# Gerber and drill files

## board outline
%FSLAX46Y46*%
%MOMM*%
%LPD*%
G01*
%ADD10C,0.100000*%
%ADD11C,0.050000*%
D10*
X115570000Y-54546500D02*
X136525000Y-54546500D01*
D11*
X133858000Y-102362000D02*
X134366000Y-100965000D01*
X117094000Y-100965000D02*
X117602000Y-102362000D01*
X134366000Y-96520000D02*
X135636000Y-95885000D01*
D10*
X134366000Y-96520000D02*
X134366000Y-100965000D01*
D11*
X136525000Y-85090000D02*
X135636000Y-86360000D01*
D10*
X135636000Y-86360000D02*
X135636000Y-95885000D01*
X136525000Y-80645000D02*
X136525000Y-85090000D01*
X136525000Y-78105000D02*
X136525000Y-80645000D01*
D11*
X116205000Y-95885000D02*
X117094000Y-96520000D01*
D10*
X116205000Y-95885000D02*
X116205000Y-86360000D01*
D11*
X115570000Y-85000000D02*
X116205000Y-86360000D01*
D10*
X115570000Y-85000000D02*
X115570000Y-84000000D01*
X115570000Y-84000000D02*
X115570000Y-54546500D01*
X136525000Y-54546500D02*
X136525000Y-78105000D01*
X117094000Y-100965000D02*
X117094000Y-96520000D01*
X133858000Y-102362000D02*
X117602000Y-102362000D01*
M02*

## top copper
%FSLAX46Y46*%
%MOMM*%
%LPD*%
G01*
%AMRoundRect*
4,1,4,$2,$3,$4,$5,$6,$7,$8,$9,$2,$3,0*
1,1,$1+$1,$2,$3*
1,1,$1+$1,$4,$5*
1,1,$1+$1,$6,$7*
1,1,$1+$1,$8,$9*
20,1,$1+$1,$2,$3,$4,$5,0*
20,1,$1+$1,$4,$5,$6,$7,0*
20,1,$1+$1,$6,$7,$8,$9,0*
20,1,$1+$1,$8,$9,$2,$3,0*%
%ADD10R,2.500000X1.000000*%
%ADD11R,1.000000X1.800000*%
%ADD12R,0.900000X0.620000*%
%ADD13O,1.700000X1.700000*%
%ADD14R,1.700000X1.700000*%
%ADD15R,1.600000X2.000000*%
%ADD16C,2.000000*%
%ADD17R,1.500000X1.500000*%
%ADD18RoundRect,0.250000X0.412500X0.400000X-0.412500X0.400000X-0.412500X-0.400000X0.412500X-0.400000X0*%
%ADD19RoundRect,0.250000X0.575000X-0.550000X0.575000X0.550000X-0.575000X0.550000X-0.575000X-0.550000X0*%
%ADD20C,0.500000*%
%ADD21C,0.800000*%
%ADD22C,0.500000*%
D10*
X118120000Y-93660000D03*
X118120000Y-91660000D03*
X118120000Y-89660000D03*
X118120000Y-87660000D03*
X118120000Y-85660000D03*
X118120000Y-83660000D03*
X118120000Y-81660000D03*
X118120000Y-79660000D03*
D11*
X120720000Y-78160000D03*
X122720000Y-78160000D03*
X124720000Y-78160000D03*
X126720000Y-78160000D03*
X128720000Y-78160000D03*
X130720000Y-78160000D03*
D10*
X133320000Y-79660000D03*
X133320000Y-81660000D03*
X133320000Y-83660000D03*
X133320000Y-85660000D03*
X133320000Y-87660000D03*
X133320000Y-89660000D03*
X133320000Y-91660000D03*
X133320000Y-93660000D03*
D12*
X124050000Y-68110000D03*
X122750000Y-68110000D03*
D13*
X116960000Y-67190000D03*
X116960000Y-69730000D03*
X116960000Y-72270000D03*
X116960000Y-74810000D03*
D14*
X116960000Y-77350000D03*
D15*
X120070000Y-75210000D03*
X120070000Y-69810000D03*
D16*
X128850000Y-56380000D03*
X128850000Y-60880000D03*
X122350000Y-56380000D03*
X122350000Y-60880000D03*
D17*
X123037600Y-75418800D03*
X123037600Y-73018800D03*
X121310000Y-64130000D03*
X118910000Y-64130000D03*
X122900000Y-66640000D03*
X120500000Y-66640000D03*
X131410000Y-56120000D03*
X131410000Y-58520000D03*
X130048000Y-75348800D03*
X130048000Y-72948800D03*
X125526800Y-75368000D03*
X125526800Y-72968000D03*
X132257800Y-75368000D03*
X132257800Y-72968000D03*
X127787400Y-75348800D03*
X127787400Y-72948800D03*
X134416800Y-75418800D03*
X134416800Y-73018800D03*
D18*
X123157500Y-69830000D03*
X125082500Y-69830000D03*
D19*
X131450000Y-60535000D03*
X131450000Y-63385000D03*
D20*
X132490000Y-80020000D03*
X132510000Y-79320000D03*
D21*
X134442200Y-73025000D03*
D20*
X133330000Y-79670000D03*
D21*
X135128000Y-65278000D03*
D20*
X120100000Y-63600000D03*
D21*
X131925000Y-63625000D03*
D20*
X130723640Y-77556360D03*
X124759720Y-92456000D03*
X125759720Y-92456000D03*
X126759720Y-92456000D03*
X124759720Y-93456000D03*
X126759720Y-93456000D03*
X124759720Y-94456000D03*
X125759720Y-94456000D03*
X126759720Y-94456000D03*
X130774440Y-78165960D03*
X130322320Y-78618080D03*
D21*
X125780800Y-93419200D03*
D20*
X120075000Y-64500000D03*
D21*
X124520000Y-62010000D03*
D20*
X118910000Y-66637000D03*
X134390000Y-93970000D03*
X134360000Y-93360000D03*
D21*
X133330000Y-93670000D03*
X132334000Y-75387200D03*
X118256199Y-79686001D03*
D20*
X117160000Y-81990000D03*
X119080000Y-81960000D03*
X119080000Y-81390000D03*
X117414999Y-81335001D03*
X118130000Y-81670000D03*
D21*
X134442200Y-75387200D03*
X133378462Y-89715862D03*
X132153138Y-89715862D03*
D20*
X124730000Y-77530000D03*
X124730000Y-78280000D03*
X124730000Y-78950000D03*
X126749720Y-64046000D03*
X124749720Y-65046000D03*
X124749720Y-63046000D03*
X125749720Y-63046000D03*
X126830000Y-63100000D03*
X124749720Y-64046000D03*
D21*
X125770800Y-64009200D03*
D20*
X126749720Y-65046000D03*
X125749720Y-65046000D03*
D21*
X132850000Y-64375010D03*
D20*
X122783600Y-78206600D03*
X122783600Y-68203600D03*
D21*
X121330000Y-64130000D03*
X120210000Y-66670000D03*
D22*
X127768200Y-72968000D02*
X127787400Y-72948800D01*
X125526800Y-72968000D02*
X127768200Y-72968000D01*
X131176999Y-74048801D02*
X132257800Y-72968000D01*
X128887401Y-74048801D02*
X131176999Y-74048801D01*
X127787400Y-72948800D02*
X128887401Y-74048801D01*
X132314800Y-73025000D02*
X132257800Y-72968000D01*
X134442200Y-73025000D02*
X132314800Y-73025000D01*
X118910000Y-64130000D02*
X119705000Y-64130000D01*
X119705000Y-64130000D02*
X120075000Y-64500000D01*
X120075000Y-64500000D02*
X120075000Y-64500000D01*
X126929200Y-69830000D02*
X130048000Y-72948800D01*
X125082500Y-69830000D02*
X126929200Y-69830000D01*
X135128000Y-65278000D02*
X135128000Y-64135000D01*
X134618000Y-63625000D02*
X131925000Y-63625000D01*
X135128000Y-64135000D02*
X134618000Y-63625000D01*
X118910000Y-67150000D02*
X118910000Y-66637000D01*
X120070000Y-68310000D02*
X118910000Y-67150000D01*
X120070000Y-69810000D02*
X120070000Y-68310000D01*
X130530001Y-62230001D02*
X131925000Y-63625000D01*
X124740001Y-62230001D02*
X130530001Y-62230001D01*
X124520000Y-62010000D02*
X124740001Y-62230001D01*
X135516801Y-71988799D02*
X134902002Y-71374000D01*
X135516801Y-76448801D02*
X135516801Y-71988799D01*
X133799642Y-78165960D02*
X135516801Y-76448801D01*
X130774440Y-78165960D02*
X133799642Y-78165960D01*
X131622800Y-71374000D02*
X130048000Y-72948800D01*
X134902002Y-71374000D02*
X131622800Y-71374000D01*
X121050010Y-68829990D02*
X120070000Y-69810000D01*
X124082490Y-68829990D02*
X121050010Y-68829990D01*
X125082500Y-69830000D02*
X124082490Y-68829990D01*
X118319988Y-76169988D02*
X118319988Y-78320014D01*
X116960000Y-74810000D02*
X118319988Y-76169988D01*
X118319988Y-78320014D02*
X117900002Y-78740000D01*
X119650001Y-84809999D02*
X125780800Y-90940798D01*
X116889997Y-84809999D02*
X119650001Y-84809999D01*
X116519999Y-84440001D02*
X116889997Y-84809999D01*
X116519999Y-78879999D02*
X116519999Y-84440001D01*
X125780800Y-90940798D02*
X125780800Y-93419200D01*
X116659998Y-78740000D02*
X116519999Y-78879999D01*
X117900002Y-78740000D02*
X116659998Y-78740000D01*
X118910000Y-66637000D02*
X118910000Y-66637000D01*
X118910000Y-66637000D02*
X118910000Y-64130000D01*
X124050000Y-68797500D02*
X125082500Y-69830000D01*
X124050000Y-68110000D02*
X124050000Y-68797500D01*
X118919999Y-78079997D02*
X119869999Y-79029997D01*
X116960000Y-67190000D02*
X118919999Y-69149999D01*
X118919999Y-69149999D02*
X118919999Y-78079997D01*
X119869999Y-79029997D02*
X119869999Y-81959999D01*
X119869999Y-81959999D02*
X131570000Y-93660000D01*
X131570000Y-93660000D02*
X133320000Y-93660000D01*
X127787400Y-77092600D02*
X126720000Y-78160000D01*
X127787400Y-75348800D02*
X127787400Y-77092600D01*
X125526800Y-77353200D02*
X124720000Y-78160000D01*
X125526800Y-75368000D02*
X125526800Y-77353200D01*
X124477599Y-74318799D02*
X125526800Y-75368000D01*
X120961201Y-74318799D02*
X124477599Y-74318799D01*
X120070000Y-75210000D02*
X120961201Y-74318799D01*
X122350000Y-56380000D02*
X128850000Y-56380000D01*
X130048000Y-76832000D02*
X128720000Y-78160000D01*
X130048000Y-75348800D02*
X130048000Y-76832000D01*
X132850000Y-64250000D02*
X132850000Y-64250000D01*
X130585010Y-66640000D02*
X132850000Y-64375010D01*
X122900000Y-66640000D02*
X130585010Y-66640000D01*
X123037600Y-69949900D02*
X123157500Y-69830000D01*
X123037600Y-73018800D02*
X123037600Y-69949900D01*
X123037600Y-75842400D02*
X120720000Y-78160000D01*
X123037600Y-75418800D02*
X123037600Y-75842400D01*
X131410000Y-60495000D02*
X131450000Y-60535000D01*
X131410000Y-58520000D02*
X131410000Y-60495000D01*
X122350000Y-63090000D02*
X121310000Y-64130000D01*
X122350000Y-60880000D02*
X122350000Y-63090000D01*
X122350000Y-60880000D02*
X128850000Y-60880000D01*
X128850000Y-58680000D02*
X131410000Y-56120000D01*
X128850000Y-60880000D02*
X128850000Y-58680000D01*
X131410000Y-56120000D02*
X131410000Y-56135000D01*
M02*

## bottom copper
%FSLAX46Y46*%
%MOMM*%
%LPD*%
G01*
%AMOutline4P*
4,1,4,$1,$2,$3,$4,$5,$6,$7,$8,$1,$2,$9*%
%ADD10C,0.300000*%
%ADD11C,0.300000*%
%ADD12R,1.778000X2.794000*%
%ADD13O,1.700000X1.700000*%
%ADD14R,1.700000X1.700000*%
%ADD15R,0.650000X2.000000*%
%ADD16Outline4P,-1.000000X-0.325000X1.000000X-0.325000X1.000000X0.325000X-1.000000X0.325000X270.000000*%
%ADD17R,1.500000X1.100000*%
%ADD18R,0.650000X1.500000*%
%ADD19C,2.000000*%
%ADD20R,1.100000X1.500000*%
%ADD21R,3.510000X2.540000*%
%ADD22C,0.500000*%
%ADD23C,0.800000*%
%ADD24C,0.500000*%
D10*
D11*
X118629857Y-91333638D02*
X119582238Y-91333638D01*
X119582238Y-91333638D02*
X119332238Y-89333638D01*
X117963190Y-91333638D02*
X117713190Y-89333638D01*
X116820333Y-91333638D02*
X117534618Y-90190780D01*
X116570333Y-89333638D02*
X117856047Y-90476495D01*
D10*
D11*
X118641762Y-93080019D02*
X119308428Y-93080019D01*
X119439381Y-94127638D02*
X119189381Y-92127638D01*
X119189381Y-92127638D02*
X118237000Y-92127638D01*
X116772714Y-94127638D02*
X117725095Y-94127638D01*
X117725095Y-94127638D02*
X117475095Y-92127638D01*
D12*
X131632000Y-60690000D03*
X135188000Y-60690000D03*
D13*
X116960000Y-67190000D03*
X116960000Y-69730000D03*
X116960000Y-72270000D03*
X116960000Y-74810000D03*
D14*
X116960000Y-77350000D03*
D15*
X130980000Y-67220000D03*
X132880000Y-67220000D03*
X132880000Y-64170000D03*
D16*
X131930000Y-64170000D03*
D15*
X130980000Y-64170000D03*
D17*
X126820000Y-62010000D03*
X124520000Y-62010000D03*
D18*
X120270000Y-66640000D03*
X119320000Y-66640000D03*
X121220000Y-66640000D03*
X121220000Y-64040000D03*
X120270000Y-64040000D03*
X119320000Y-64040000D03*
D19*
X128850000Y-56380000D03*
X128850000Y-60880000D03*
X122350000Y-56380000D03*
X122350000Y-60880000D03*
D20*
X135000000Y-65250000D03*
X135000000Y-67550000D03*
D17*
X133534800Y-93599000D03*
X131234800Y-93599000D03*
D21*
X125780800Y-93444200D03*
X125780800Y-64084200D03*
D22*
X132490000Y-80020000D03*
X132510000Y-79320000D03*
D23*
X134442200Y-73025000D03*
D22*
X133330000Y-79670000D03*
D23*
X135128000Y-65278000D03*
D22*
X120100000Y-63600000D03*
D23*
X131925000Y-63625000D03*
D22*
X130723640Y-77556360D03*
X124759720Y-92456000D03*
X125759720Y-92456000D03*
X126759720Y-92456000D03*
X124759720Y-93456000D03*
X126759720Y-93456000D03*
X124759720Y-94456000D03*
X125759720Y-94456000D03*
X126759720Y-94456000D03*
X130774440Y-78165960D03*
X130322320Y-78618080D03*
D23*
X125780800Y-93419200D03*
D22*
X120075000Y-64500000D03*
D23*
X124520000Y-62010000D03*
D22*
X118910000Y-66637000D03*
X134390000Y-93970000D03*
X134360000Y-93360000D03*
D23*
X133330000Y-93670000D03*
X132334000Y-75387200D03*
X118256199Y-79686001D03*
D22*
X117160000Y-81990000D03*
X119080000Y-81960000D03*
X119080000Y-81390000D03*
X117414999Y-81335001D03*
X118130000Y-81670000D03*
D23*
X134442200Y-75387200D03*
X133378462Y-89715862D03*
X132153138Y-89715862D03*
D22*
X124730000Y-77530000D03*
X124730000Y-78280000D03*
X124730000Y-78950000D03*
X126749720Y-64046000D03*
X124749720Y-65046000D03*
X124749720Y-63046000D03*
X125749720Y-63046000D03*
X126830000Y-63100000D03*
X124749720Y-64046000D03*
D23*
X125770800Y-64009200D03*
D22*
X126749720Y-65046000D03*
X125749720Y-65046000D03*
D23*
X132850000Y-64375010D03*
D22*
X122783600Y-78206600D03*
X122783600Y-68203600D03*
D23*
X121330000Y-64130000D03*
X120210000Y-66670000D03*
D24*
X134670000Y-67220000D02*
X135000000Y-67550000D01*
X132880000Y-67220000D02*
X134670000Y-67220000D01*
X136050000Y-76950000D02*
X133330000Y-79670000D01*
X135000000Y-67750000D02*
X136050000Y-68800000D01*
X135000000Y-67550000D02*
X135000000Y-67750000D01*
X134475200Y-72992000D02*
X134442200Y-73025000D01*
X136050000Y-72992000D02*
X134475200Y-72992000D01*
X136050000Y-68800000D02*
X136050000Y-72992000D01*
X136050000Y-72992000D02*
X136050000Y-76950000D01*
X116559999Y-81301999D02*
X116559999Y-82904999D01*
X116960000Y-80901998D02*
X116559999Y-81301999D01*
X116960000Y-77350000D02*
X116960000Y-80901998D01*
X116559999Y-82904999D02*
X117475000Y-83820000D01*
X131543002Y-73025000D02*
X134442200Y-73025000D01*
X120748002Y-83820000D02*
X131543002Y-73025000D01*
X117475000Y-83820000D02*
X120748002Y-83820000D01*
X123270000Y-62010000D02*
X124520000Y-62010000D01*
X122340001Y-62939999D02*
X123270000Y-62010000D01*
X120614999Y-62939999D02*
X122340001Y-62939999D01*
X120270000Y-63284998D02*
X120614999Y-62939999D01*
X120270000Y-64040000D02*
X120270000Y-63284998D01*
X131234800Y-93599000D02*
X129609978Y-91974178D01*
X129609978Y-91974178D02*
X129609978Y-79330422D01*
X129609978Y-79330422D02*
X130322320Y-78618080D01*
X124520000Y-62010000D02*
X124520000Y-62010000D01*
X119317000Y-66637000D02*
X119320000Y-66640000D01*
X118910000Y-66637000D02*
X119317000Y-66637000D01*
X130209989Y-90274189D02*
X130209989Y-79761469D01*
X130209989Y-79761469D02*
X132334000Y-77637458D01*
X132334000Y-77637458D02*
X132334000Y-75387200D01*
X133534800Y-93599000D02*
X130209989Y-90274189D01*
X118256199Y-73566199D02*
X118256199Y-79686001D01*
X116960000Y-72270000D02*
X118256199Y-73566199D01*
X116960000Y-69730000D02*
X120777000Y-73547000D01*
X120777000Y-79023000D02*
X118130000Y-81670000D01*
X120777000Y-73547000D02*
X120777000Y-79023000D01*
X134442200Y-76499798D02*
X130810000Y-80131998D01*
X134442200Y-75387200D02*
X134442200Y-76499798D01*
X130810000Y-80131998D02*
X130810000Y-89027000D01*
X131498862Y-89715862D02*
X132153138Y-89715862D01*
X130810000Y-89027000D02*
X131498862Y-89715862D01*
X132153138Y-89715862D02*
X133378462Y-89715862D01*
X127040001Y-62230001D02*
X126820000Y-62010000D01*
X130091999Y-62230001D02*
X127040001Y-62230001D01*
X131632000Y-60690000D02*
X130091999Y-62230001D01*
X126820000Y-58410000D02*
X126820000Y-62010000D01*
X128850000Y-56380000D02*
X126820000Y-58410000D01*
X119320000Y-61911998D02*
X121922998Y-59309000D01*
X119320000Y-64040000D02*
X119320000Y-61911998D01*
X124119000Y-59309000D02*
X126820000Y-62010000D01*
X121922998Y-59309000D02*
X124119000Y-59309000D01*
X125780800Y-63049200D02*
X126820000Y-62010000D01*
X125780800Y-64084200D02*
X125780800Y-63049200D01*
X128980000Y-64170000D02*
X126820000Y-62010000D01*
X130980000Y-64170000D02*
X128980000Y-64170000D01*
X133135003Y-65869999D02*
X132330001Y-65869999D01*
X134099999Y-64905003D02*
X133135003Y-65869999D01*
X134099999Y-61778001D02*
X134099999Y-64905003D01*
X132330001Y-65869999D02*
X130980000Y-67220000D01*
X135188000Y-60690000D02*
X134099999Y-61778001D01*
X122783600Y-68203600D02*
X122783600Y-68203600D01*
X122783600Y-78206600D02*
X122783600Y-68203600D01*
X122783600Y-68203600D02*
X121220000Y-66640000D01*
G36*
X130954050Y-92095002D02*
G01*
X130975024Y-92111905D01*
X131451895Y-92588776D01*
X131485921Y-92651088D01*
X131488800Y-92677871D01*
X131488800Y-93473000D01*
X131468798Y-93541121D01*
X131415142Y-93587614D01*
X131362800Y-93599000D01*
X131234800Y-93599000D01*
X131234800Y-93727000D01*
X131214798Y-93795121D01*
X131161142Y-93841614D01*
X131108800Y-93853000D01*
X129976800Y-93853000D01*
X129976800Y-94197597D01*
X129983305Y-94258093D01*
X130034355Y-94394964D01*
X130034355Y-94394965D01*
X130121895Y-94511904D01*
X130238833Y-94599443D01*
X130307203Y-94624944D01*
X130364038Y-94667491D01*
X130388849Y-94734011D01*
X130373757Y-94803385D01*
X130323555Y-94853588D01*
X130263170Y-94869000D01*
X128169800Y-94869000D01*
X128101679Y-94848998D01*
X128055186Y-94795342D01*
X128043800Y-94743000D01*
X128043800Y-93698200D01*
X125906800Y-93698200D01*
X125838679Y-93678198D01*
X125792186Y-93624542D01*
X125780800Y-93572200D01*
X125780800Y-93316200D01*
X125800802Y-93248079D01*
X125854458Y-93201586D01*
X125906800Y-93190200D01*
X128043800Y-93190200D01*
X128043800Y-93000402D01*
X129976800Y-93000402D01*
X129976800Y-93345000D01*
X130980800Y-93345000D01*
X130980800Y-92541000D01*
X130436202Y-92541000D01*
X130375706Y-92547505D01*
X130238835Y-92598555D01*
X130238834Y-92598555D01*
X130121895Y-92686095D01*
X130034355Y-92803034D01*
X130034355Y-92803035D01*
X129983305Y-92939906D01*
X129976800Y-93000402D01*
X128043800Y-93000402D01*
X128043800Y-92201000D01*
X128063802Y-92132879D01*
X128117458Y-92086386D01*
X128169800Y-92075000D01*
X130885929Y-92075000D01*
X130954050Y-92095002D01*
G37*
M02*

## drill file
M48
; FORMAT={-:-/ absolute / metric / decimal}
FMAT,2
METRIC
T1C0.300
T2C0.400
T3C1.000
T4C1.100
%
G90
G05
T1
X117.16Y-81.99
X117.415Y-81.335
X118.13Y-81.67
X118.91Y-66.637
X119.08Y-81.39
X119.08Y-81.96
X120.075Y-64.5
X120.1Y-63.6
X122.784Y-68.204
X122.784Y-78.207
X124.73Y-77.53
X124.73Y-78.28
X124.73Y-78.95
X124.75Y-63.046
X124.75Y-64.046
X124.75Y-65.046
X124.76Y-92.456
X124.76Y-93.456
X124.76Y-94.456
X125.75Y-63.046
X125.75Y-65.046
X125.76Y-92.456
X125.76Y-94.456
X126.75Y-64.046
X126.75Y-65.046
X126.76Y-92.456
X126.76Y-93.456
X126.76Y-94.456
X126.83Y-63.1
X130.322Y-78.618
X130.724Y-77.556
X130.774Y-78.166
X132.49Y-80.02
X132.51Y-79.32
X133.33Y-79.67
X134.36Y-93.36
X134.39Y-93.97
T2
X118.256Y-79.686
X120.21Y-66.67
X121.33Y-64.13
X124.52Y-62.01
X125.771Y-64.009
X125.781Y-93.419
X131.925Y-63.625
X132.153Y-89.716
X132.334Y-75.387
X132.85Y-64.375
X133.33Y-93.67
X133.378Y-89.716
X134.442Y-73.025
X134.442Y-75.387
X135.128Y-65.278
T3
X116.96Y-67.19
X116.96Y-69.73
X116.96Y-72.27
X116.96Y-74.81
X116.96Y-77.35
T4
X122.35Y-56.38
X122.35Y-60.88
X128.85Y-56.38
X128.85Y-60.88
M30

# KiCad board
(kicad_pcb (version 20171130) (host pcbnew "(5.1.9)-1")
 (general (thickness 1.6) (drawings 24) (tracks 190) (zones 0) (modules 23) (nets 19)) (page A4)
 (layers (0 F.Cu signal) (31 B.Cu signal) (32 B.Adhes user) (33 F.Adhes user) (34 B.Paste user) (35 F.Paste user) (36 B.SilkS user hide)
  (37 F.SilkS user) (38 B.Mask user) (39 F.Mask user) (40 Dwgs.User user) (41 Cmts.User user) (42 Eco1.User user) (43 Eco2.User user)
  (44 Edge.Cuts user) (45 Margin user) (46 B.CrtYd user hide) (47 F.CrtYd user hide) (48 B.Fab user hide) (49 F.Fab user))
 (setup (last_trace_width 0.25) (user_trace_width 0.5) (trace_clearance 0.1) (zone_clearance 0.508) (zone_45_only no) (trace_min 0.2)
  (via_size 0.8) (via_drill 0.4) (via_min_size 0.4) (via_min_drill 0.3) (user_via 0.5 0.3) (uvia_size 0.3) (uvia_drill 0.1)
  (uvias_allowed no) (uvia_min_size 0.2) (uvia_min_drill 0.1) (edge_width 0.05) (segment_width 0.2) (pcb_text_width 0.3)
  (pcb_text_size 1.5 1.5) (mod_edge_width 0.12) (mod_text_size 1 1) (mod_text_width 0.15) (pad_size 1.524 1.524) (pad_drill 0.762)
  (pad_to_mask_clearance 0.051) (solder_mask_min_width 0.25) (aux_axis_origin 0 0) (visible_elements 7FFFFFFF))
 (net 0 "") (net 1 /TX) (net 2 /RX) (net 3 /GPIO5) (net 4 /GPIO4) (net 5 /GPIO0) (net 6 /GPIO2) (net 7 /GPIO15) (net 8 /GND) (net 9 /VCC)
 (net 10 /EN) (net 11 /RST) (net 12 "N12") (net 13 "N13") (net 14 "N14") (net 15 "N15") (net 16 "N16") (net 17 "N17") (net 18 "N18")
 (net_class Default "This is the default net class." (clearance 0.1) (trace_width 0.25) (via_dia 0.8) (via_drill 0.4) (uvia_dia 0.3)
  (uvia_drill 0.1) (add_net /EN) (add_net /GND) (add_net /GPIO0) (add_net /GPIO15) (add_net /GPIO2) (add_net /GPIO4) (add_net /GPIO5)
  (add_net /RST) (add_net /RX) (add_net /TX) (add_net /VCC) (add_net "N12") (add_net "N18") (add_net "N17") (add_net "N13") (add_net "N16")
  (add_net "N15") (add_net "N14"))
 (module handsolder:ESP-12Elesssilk (layer F.Cu) (at 125.72 90.16 180)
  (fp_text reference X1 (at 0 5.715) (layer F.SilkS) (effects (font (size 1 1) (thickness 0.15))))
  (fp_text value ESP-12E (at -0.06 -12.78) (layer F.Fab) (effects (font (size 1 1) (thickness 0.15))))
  (pad 22 smd rect (at 7.6 -3.5 180) (size 2.5 1) (layers F.Cu F.Paste F.Mask))
  (pad 21 smd rect (at 7.6 -1.5 180) (size 2.5 1) (layers F.Cu F.Paste F.Mask))
  (pad 20 smd rect (at 7.6 0.5 180) (size 2.5 1) (layers F.Cu F.Paste F.Mask))
  (pad 19 smd rect (at 7.6 2.5 180) (size 2.5 1) (layers F.Cu F.Paste F.Mask))
  (pad 18 smd rect (at 7.6 4.5 180) (size 2.5 1) (layers F.Cu F.Paste F.Mask))
  (pad 17 smd rect (at 7.6 6.5 180) (size 2.5 1) (layers F.Cu F.Paste F.Mask))
  (pad 16 smd rect (at 7.6 8.5 180) (size 2.5 1) (layers F.Cu F.Paste F.Mask) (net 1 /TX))
  (pad 15 smd rect (at 7.6 10.5 180) (size 2.5 1) (layers F.Cu F.Paste F.Mask) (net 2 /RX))
  (pad 14 smd rect (at 5 12 180) (size 1 1.8) (layers F.Cu F.Paste F.Mask) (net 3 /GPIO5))
  (pad 13 smd rect (at 3 12 180) (size 1 1.8) (layers F.Cu F.Paste F.Mask) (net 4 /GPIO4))
  (pad 12 smd rect (at 1 12 180) (size 1 1.8) (layers F.Cu F.Paste F.Mask) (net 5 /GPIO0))
  (pad 11 smd rect (at -1 12 180) (size 1 1.8) (layers F.Cu F.Paste F.Mask) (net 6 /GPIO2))
  (pad 10 smd rect (at -3 12 180) (size 1 1.8) (layers F.Cu F.Paste F.Mask) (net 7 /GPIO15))
  (pad 9 smd rect (at -5 12 180) (size 1 1.8) (layers F.Cu F.Paste F.Mask) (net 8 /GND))
  (pad 8 smd rect (at -7.6 10.5 180) (size 2.5 1) (layers F.Cu F.Paste F.Mask) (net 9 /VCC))
  (pad 7 smd rect (at -7.6 8.5 180) (size 2.5 1) (layers F.Cu F.Paste F.Mask))
  (pad 6 smd rect (at -7.6 6.5 180) (size 2.5 1) (layers F.Cu F.Paste F.Mask))
  (pad 5 smd rect (at -7.6 4.5 180) (size 2.5 1) (layers F.Cu F.Paste F.Mask))
  (pad 4 smd rect (at -7.6 2.5 180) (size 2.5 1) (layers F.Cu F.Paste F.Mask))
  (pad 3 smd rect (at -7.6 0.5 180) (size 2.5 1) (layers F.Cu F.Paste F.Mask) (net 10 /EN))
  (pad 2 smd rect (at -7.6 -1.5 180) (size 2.5 1) (layers F.Cu F.Paste F.Mask))
  (pad 1 smd rect (at -7.6 -3.5 180) (size 2.5 1) (layers F.Cu F.Paste F.Mask) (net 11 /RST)))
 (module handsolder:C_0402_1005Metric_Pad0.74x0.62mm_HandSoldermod (layer F.Cu) (at 123.4 68.11)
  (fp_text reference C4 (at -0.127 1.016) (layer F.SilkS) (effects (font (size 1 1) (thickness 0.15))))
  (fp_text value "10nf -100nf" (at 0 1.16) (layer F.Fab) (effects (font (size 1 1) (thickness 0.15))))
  (pad 2 smd rect (at 0.65 0) (size 0.9 0.62) (layers F.Cu F.Paste F.Mask) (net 8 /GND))
  (pad 1 smd rect (at -0.65 0) (size 0.9 0.62) (layers F.Cu F.Paste F.Mask) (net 4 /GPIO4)))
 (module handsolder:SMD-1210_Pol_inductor (layer B.Cu) (at 133.41 60.69)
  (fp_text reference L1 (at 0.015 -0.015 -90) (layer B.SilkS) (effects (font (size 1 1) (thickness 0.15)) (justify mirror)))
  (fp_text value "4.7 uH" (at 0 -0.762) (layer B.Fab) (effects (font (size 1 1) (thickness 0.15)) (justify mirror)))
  (pad 1 smd rect (at -1.778 0) (size 1.778 2.794) (layers B.Cu B.Paste B.Mask) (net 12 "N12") (zone_connect 2))
  (pad 2 smd rect (at 1.778 0) (size 1.778 2.794) (layers B.Cu B.Paste B.Mask) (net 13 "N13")))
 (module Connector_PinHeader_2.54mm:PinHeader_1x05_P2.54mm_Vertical (layer F.Cu) (at 116.96 77.35 180)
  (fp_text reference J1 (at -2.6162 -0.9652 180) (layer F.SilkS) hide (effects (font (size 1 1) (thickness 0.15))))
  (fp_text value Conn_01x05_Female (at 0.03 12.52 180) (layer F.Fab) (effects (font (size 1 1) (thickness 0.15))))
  (pad 5 thru_hole oval (at 0 10.16 180) (size 1.7 1.7) (drill 1) (layers *.Cu *.Mask) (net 11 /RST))
  (pad 4 thru_hole oval (at 0 7.62 180) (size 1.7 1.7) (drill 1) (layers *.Cu *.Mask) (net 1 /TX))
  (pad 3 thru_hole oval (at 0 5.08 180) (size 1.7 1.7) (drill 1) (layers *.Cu *.Mask) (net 2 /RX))
  (pad 2 thru_hole oval (at 0 2.54 180) (size 1.7 1.7) (drill 1) (layers *.Cu *.Mask) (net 8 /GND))
  (pad 1 thru_hole rect (at 0 0 180) (size 1.7 1.7) (drill 1) (layers *.Cu *.Mask) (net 9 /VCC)))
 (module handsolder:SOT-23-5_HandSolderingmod (layer B.Cu) (at 131.93 65.72 270)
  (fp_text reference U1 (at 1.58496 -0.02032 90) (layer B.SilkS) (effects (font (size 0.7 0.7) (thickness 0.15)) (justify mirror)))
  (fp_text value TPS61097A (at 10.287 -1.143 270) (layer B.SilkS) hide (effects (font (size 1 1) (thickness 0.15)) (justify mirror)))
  (pad 5 smd rect (at 1.5 0.95 270) (size 2 0.65) (layers B.Cu B.Paste B.Mask) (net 13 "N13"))
  (pad 4 smd rect (at 1.5 -0.95 270) (size 2 0.65) (layers B.Cu B.Paste B.Mask) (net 9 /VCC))
  (pad 3 smd rect (at -1.55 -0.95 270) (size 2 0.65) (layers B.Cu B.Paste B.Mask) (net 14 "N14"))
  (pad 2 smd trapezoid (at -1.55 0 270) (size 2 0.65) (layers B.Cu B.Paste B.Mask) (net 8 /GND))
  (pad 1 smd rect (at -1.55 0.95 270) (size 2 0.65) (layers B.Cu B.Paste B.Mask) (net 12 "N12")))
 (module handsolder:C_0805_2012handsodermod (layer B.Cu) (at 125.67 62.01)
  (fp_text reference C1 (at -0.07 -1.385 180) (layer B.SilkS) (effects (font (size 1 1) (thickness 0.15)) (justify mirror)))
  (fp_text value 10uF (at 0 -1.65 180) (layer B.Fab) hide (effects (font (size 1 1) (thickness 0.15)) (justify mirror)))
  (pad 2 smd rect (at 1.15 0) (size 1.5 1.1) (layers B.Cu B.Paste B.Mask) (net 12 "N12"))
  (pad 1 smd rect (at -1.15 0) (size 1.5 1.1) (layers B.Cu B.Paste B.Mask) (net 8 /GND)))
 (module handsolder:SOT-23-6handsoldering (layer B.Cu) (at 120.27 65.34 270)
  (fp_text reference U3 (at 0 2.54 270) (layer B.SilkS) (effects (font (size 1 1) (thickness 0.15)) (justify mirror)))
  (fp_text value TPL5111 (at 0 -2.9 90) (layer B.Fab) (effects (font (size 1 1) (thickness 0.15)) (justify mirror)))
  (pad 5 smd rect (at 1.3 0 270) (size 1.5 0.65) (layers B.Cu B.Paste B.Mask) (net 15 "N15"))
  (pad 6 smd rect (at 1.3 0.95 270) (size 1.5 0.65) (layers B.Cu B.Paste B.Mask) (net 8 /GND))
  (pad 4 smd rect (at 1.3 -0.95 270) (size 1.5 0.65) (layers B.Cu B.Paste B.Mask) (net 4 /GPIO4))
  (pad 3 smd rect (at -1.3 -0.95 270) (size 1.5 0.65) (layers B.Cu B.Paste B.Mask) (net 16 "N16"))
  (pad 2 smd rect (at -1.3 0 270) (size 1.5 0.65) (layers B.Cu B.Paste B.Mask) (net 8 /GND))
  (pad 1 smd rect (at -1.3 0.95 270) (size 1.5 0.65) (layers B.Cu B.Paste B.Mask) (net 12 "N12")))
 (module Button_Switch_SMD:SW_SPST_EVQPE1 (layer F.Cu) (at 120.07 72.51 90)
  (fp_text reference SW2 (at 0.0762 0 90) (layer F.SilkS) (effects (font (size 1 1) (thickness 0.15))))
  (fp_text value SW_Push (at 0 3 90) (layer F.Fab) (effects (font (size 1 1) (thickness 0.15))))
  (pad 1 smd rect (at -2.7 0 90) (size 2 1.6) (layers F.Cu F.Paste F.Mask) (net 5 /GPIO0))
  (pad 2 smd rect (at 2.7 0 90) (size 2 1.6) (layers F.Cu F.Paste F.Mask) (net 8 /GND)))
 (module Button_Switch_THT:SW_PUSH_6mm (layer F.Cu) (at 122.35 56.38)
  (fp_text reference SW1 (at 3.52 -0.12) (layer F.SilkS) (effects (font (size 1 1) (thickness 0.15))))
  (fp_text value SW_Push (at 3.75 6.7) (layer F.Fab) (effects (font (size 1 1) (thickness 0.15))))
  (pad 1 thru_hole circle (at 6.5 0 90) (size 2 2) (drill 1.1) (layers *.Cu *.Mask) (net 12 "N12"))
  (pad 2 thru_hole circle (at 6.5 4.5 90) (size 2 2) (drill 1.1) (layers *.Cu *.Mask) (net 16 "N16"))
  (pad 1 thru_hole circle (at 0 0 90) (size 2 2) (drill 1.1) (layers *.Cu *.Mask) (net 12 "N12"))
  (pad 2 thru_hole circle (at 0 4.5 90) (size 2 2) (drill 1.1) (layers *.Cu *.Mask) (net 16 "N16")))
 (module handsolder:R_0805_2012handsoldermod (layer F.Cu) (at 123.0376 74.2188 270)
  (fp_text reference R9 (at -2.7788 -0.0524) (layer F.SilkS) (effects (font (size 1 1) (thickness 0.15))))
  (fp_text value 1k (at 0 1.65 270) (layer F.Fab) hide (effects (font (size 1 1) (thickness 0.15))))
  (pad 2 smd rect (at 1.2 0 270) (size 1.5 1.5) (layers F.Cu F.Paste F.Mask) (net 3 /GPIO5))
  (pad 1 smd rect (at -1.2 0 270) (size 1.5 1.5) (layers F.Cu F.Paste F.Mask) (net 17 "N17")))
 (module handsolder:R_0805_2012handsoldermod (layer F.Cu) (at 120.11 64.13)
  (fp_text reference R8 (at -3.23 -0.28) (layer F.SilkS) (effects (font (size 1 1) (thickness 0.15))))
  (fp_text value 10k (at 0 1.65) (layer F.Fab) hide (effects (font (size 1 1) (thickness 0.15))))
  (pad 2 smd rect (at 1.2 0) (size 1.5 1.5) (layers F.Cu F.Paste F.Mask) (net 16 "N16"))
  (pad 1 smd rect (at -1.2 0) (size 1.5 1.5) (layers F.Cu F.Paste F.Mask) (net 8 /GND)))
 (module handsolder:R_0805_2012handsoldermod (layer F.Cu) (at 121.7 66.64)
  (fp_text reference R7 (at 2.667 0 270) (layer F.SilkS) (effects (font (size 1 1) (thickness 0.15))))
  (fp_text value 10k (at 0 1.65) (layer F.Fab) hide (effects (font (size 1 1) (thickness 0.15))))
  (pad 2 smd rect (at 1.2 0) (size 1.5 1.5) (layers F.Cu F.Paste F.Mask) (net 14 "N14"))
  (pad 1 smd rect (at -1.2 0) (size 1.5 1.5) (layers F.Cu F.Paste F.Mask) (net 15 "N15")))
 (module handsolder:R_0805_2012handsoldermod (layer F.Cu) (at 131.41 57.32 90)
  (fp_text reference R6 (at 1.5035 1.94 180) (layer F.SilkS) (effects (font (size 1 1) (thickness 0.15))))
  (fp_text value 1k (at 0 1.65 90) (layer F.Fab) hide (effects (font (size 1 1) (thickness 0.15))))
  (pad 2 smd rect (at 1.2 0 90) (size 1.5 1.5) (layers F.Cu F.Paste F.Mask) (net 16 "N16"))
  (pad 1 smd rect (at -1.2 0 90) (size 1.5 1.5) (layers F.Cu F.Paste F.Mask) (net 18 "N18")))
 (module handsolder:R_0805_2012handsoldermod (layer F.Cu) (at 130.048 74.1488 270)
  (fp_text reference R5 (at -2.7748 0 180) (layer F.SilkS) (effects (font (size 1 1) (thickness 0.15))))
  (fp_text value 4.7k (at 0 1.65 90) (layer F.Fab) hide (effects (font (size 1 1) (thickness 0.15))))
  (pad 2 smd rect (at 1.2 0 270) (size 1.5 1.5) (layers F.Cu F.Paste F.Mask) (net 7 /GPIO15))
  (pad 1 smd rect (at -1.2 0 270) (size 1.5 1.5) (layers F.Cu F.Paste F.Mask) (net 8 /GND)))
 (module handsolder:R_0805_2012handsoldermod (layer F.Cu) (at 125.5268 74.168 270)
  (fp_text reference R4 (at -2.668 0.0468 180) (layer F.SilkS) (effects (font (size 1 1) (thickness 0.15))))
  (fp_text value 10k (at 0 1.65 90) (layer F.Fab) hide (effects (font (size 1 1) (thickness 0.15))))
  (pad 2 smd rect (at 1.2 0 270) (size 1.5 1.5) (layers F.Cu F.Paste F.Mask) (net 5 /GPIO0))
  (pad 1 smd rect (at -1.2 0 270) (size 1.5 1.5) (layers F.Cu F.Paste F.Mask) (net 9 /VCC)))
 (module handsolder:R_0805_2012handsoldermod (layer F.Cu) (at 132.2578 74.168 270)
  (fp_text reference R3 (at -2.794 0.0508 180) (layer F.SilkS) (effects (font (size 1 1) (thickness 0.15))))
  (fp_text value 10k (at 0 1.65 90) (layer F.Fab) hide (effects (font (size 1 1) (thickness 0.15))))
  (pad 2 smd rect (at 1.2 0 270) (size 1.5 1.5) (layers F.Cu F.Paste F.Mask) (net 11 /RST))
  (pad 1 smd rect (at -1.2 0 270) (size 1.5 1.5) (layers F.Cu F.Paste F.Mask) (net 9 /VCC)))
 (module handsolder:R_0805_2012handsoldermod (layer F.Cu) (at 127.7874 74.1488 270)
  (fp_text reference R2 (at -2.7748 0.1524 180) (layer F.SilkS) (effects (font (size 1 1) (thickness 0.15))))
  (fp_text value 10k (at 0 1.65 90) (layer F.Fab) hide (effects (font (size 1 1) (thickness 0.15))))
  (pad 2 smd rect (at 1.2 0 270) (size 1.5 1.5) (layers F.Cu F.Paste F.Mask) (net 6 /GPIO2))
  (pad 1 smd rect (at -1.2 0 270) (size 1.5 1.5) (layers F.Cu F.Paste F.Mask) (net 9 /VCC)))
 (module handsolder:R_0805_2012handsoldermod (layer F.Cu) (at 134.4168 74.2188 270)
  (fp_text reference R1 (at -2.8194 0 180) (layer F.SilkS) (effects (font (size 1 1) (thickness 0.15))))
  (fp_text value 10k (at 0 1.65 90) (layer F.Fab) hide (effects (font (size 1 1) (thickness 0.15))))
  (pad 2 smd rect (at 1.2 0 270) (size 1.5 1.5) (layers F.Cu F.Paste F.Mask) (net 10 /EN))
  (pad 1 smd rect (at -1.2 0 270) (size 1.5 1.5) (layers F.Cu F.Paste F.Mask) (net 9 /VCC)))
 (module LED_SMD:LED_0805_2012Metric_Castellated (layer F.Cu) (at 124.12 69.83 180)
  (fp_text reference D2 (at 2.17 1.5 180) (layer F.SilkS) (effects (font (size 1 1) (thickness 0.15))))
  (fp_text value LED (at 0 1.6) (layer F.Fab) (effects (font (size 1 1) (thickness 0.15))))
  (pad 2 smd roundrect (at 0.9625 0 180) (size 1.325 1.3) (layers F.Cu F.Paste F.Mask) (roundrect_rratio 0.1923076923076923) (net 17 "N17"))
  (pad 1 smd roundrect (at -0.9625 0 180) (size 1.325 1.3) (layers F.Cu F.Paste F.Mask) (roundrect_rratio 0.1923076923076923) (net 8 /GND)))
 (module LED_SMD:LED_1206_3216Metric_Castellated (layer F.Cu) (at 131.45 61.96 90)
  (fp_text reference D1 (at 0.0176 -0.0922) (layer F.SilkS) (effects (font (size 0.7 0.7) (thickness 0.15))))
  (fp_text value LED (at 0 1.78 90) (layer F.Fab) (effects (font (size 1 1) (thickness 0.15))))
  (pad 2 smd roundrect (at 1.425 0 90) (size 1.6 1.65) (layers F.Cu F.Paste F.Mask) (roundrect_rratio 0.15625) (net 18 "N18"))
  (pad 1 smd roundrect (at -1.425 0 90) (size 1.6 1.65) (layers F.Cu F.Paste F.Mask) (roundrect_rratio 0.15625) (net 8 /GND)))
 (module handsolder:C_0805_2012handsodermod (layer B.Cu) (at 135 66.4 90)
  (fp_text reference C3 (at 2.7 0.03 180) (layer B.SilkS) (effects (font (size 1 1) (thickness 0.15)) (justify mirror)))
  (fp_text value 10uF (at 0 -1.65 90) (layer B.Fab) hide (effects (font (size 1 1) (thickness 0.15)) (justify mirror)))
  (pad 2 smd rect (at 1.15 0 90) (size 1.5 1.1) (layers B.Cu B.Paste B.Mask) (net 8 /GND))
  (pad 1 smd rect (at -1.15 0 90) (size 1.5 1.1) (layers B.Cu B.Paste B.Mask) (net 9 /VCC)))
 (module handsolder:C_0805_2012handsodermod (layer B.Cu) (at 132.3848 93.599)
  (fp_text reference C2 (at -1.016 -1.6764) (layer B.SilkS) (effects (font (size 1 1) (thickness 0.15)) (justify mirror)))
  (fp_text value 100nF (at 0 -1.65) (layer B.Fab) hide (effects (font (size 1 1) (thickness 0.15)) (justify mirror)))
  (pad 2 smd rect (at 1.15 0) (size 1.5 1.1) (layers B.Cu B.Paste B.Mask) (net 11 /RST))
  (pad 1 smd rect (at -1.15 0) (size 1.5 1.1) (layers B.Cu B.Paste B.Mask) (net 8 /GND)))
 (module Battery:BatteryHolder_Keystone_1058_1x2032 (layer B.Cu) (at 125.7808 78.7642 270)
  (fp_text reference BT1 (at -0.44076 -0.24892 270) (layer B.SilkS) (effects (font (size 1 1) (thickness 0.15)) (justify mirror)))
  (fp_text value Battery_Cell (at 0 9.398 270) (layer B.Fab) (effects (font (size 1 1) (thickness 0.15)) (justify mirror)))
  (pad 2 smd rect (at 14.68 0 270) (size 2.54 3.51) (layers B.Cu B.Paste B.Mask) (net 8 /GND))
  (pad 1 smd rect (at -14.68 0 270) (size 2.54 3.51) (layers B.Cu B.Paste B.Mask) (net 12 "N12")))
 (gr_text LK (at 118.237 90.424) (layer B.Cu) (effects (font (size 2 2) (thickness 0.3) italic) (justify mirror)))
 (gr_line (start 115.57 54.5465) (end 136.525 54.5465) (layer Edge.Cuts) (width 0.1))
 (gr_line (start 133.858 102.362) (end 134.366 100.965) (layer Edge.Cuts) (width 0.05))
 (gr_line (start 117.094 100.965) (end 117.602 102.362) (layer Edge.Cuts) (width 0.05))
 (gr_line (start 134.366 96.52) (end 135.636 95.885) (layer Edge.Cuts) (width 0.05))
 (gr_line (start 134.366 96.52) (end 134.366 100.965) (layer Edge.Cuts) (width 0.1))
 (gr_line (start 136.525 85.09) (end 135.636 86.36) (layer Edge.Cuts) (width 0.05))
 (gr_line (start 135.636 86.36) (end 135.636 95.885) (layer Edge.Cuts) (width 0.1))
 (gr_line (start 136.525 80.645) (end 136.525 85.09) (layer Edge.Cuts) (width 0.1))
 (gr_line (start 136.525 78.105) (end 136.525 80.645) (layer Edge.Cuts) (width 0.1))
 (gr_line (start 116.205 95.885) (end 117.094 96.52) (layer Edge.Cuts) (width 0.05))
 (gr_line (start 116.205 95.885) (end 116.205 86.36) (layer Edge.Cuts) (width 0.1))
 (gr_line (start 115.57 85) (end 116.205 86.36) (layer Edge.Cuts) (width 0.05))
 (gr_line (start 115.57 85) (end 115.57 84) (layer Edge.Cuts) (width 0.1))
 (gr_line (start 115.57 84) (end 115.57 54.5465) (layer Edge.Cuts) (width 0.1))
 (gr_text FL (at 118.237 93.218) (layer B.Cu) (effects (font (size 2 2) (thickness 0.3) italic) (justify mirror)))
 (gr_line (start 136.525 54.5465) (end 136.525 78.105) (layer Edge.Cuts) (width 0.1))
 (gr_line (start 117.094 100.965) (end 117.094 96.52) (layer Edge.Cuts) (width 0.1))
 (gr_line (start 133.858 102.362) (end 117.602 102.362) (layer Edge.Cuts) (width 0.1))
 (via (at 132.49 80.02) (size 0.5) (drill 0.3) (layers F.Cu B.Cu) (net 9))
 (via (at 132.51 79.32) (size 0.5) (drill 0.3) (layers F.Cu B.Cu) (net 9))
 (via (at 134.4422 73.025) (size 0.8) (drill 0.4) (layers F.Cu B.Cu) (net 9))
 (via (at 133.33 79.67) (size 0.5) (drill 0.3) (layers F.Cu B.Cu) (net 9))
 (segment (start 127.7682 72.968) (end 127.7874 72.9488) (width 0.5) (layer F.Cu) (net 9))
 (segment (start 125.5268 72.968) (end 127.7682 72.968) (width 0.5) (layer F.Cu) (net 9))
 (segment (start 131.176999 74.048801) (end 132.2578 72.968) (width 0.5) (layer F.Cu) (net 9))
 (segment (start 128.887401 74.048801) (end 131.176999 74.048801) (width 0.5) (layer F.Cu) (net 9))
 (segment (start 127.7874 72.9488) (end 128.887401 74.048801) (width 0.5) (layer F.Cu) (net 9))
 (segment (start 134.67 67.22) (end 135 67.55) (width 0.5) (layer B.Cu) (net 9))
 (segment (start 132.88 67.22) (end 134.67 67.22) (width 0.5) (layer B.Cu) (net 9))
 (segment (start 136.05 76.95) (end 133.33 79.67) (width 0.5) (layer B.Cu) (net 9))
 (segment (start 135 67.75) (end 136.05 68.8) (width 0.5) (layer B.Cu) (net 9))
 (segment (start 135 67.55) (end 135 67.75) (width 0.5) (layer B.Cu) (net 9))
 (segment (start 134.4752 72.992) (end 134.4422 73.025) (width 0.5) (layer B.Cu) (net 9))
 (segment (start 136.05 72.992) (end 134.4752 72.992) (width 0.5) (layer B.Cu) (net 9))
 (segment (start 136.05 68.8) (end 136.05 72.992) (width 0.5) (layer B.Cu) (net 9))
 (segment (start 136.05 72.992) (end 136.05 76.95) (width 0.5) (layer B.Cu) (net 9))
 (segment (start 132.3148 73.025) (end 132.2578 72.968) (width 0.5) (layer F.Cu) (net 9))
 (segment (start 134.4422 73.025) (end 132.3148 73.025) (width 0.5) (layer F.Cu) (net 9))
 (segment (start 116.559999 81.301999) (end 116.559999 82.904999) (width 0.5) (layer B.Cu) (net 9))
 (segment (start 116.96 80.901998) (end 116.559999 81.301999) (width 0.5) (layer B.Cu) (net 9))
 (segment (start 116.96 77.35) (end 116.96 80.901998) (width 0.5) (layer B.Cu) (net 9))
 (segment (start 116.559999 82.904999) (end 117.475 83.82) (width 0.5) (layer B.Cu) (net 9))
 (segment (start 131.543002 73.025) (end 134.4422 73.025) (width 0.5) (layer B.Cu) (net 9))
 (segment (start 120.748002 83.82) (end 131.543002 73.025) (width 0.5) (layer B.Cu) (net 9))
 (segment (start 117.475 83.82) (end 120.748002 83.82) (width 0.5) (layer B.Cu) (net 9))
 (via (at 135.128 65.278) (size 0.8) (drill 0.4) (layers F.Cu B.Cu) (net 8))
 (via (at 120.1 63.6) (size 0.5) (drill 0.3) (layers F.Cu B.Cu) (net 8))
 (via (at 131.925 63.625) (size 0.8) (drill 0.4) (layers F.Cu B.Cu) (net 8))
 (via (at 130.72364 77.55636) (size 0.5) (drill 0.3) (layers F.Cu B.Cu) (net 8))
 (via (at 124.75972 92.456) (size 0.5) (drill 0.3) (layers F.Cu B.Cu) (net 8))
 (via (at 125.75972 92.456) (size 0.5) (drill 0.3) (layers F.Cu B.Cu) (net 8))
 (via (at 126.75972 92.456) (size 0.5) (drill 0.3) (layers F.Cu B.Cu) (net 8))
 (via (at 124.75972 93.456) (size 0.5) (drill 0.3) (layers F.Cu B.Cu) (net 8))
 (via (at 126.75972 93.456) (size 0.5) (drill 0.3) (layers F.Cu B.Cu) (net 8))
 (via (at 124.75972 94.456) (size 0.5) (drill 0.3) (layers F.Cu B.Cu) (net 8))
 (via (at 125.75972 94.456) (size 0.5) (drill 0.3) (layers F.Cu B.Cu) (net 8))
 (via (at 126.75972 94.456) (size 0.5) (drill 0.3) (layers F.Cu B.Cu) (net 8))
 (via (at 130.77444 78.16596) (size 0.5) (drill 0.3) (layers F.Cu B.Cu) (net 8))
 (via (at 130.32232 78.61808) (size 0.5) (drill 0.3) (layers F.Cu B.Cu) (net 8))
 (via (at 125.7808 93.4192) (size 0.8) (drill 0.4) (layers F.Cu B.Cu) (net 8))
 (segment (start 118.91 64.13) (end 119.705 64.13) (width 0.5) (layer F.Cu) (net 8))
 (segment (start 119.705 64.13) (end 120.075 64.5) (width 0.5) (layer F.Cu) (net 8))
 (segment (start 120.075 64.5) (end 120.075 64.5) (width 0.5) (layer F.Cu) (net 8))
 (via (at 120.075 64.5) (size 0.5) (drill 0.3) (layers F.Cu B.Cu) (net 8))
 (segment (start 126.9292 69.83) (end 130.048 72.9488) (width 0.5) (layer F.Cu) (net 8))
 (segment (start 125.0825 69.83) (end 126.9292 69.83) (width 0.5) (layer F.Cu) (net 8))
 (segment (start 123.27 62.01) (end 124.52 62.01) (width 0.5) (layer B.Cu) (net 8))
 (segment (start 122.340001 62.939999) (end 123.27 62.01) (width 0.5) (layer B.Cu) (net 8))
 (segment (start 120.614999 62.939999) (end 122.340001 62.939999) (width 0.5) (layer B.Cu) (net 8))
 (segment (start 120.27 63.284998) (end 120.614999 62.939999) (width 0.5) (layer B.Cu) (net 8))
 (segment (start 120.27 64.04) (end 120.27 63.284998) (width 0.5) (layer B.Cu) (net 8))
 (segment (start 135.128 65.278) (end 135.128 64.135) (width 0.5) (layer F.Cu) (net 8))
 (segment (start 134.618 63.625) (end 131.925 63.625) (width 0.5) (layer F.Cu) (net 8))
 (segment (start 135.128 64.135) (end 134.618 63.625) (width 0.5) (layer F.Cu) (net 8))
 (segment (start 118.91 67.15) (end 118.91 66.637) (width 0.5) (layer F.Cu) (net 8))
 (segment (start 120.07 68.31) (end 118.91 67.15) (width 0.5) (layer F.Cu) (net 8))
 (segment (start 120.07 69.81) (end 120.07 68.31) (width 0.5) (layer F.Cu) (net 8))
 (segment (start 131.2348 93.599) (end 129.609978 91.974178) (width 0.5) (layer B.Cu) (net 8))
 (segment (start 129.609978 91.974178) (end 129.609978 79.330422) (width 0.5) (layer B.Cu) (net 8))
 (segment (start 129.609978 79.330422) (end 130.32232 78.61808) (width 0.5) (layer B.Cu) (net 8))
 (segment (start 124.52 62.01) (end 124.52 62.01) (width 0.5) (layer B.Cu) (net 8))
 (via (at 124.52 62.01) (size 0.8) (drill 0.4) (layers F.Cu B.Cu) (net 8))
 (segment (start 130.530001 62.230001) (end 131.925 63.625) (width 0.5) (layer F.Cu) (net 8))
 (segment (start 124.740001 62.230001) (end 130.530001 62.230001) (width 0.5) (layer F.Cu) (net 8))
 (segment (start 124.52 62.01) (end 124.740001 62.230001) (width 0.5) (layer F.Cu) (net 8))
 (segment (start 135.516801 71.988799) (end 134.902002 71.374) (width 0.5) (layer F.Cu) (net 8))
 (segment (start 135.516801 76.448801) (end 135.516801 71.988799) (width 0.5) (layer F.Cu) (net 8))
 (segment (start 133.799642 78.16596) (end 135.516801 76.448801) (width 0.5) (layer F.Cu) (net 8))
 (segment (start 130.77444 78.16596) (end 133.799642 78.16596) (width 0.5) (layer F.Cu) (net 8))
 (segment (start 131.6228 71.374) (end 130.048 72.9488) (width 0.5) (layer F.Cu) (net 8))
 (segment (start 134.902002 71.374) (end 131.6228 71.374) (width 0.5) (layer F.Cu) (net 8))
 (segment (start 121.05001 68.82999) (end 120.07 69.81) (width 0.5) (layer F.Cu) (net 8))
 (segment (start 124.08249 68.82999) (end 121.05001 68.82999) (width 0.5) (layer F.Cu) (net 8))
 (segment (start 125.0825 69.83) (end 124.08249 68.82999) (width 0.5) (layer F.Cu) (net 8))
 (segment (start 118.319988 76.169988) (end 118.319988 78.320014) (width 0.5) (layer F.Cu) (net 8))
 (segment (start 116.96 74.81) (end 118.319988 76.169988) (width 0.5) (layer F.Cu) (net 8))
 (segment (start 118.319988 78.320014) (end 117.900002 78.74) (width 0.5) (layer F.Cu) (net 8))
 (segment (start 119.650001 84.809999) (end 125.7808 90.940798) (width 0.5) (layer F.Cu) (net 8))
 (segment (start 116.889997 84.809999) (end 119.650001 84.809999) (width 0.5) (layer F.Cu) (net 8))
 (segment (start 116.519999 84.440001) (end 116.889997 84.809999) (width 0.5) (layer F.Cu) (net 8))
 (segment (start 116.519999 78.879999) (end 116.519999 84.440001) (width 0.5) (layer F.Cu) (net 8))
 (segment (start 125.7808 90.940798) (end 125.7808 93.4192) (width 0.5) (layer F.Cu) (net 8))
 (segment (start 116.659998 78.74) (end 116.519999 78.879999) (width 0.5) (layer F.Cu) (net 8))
 (segment (start 117.900002 78.74) (end 116.659998 78.74) (width 0.5) (layer F.Cu) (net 8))
 (segment (start 118.91 66.637) (end 118.91 66.637) (width 0.5) (layer F.Cu) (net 8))
 (segment (start 118.91 66.637) (end 118.91 64.13) (width 0.5) (layer F.Cu) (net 8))
 (via (at 118.91 66.637) (size 0.5) (drill 0.3) (layers F.Cu B.Cu) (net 8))
 (segment (start 119.317 66.637) (end 119.32 66.64) (width 0.5) (layer B.Cu) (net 8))
 (segment (start 118.91 66.637) (end 119.317 66.637) (width 0.5) (layer B.Cu) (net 8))
 (segment (start 124.05 68.7975) (end 125.0825 69.83) (width 0.5) (layer F.Cu) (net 8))
 (segment (start 124.05 68.11) (end 124.05 68.7975) (width 0.5) (layer F.Cu) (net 8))
 (via (at 134.39 93.97) (size 0.5) (drill 0.3) (layers F.Cu B.Cu) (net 11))
 (via (at 134.36 93.36) (size 0.5) (drill 0.3) (layers F.Cu B.Cu) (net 11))
 (via (at 133.33 93.67) (size 0.8) (drill 0.4) (layers F.Cu B.Cu) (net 11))
 (via (at 132.334 75.3872) (size 0.8) (drill 0.4) (layers F.Cu B.Cu) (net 11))
 (segment (start 130.209989 90.274189) (end 130.209989 79.761469) (width 0.5) (layer B.Cu) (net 11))
 (segment (start 130.209989 79.761469) (end 132.334 77.637458) (width 0.5) (layer B.Cu) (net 11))
 (segment (start 132.334 77.637458) (end 132.334 75.3872) (width 0.5) (layer B.Cu) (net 11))
 (segment (start 133.5348 93.599) (end 130.209989 90.274189) (width 0.5) (layer B.Cu) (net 11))
 (segment (start 118.919999 78.079997) (end 119.869999 79.029997) (width 0.5) (layer F.Cu) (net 11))
 (segment (start 116.96 67.19) (end 118.919999 69.149999) (width 0.5) (layer F.Cu) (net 11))
 (segment (start 118.919999 69.149999) (end 118.919999 78.079997) (width 0.5) (layer F.Cu) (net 11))
 (segment (start 119.869999 79.029997) (end 119.869999 81.959999) (width 0.5) (layer F.Cu) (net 11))
 (segment (start 119.869999 81.959999) (end 131.57 93.66) (width 0.5) (layer F.Cu) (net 11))
 (segment (start 131.57 93.66) (end 133.32 93.66) (width 0.5) (layer F.Cu) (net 11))
 (via (at 118.256199 79.686001) (size 0.8) (drill 0.4) (layers F.Cu B.Cu) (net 2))
 (segment (start 118.256199 73.566199) (end 118.256199 79.686001) (width 0.5) (layer B.Cu) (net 2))
 (segment (start 116.96 72.27) (end 118.256199 73.566199) (width 0.5) (layer B.Cu) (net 2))
 (via (at 117.16 81.99) (size 0.5) (drill 0.3) (layers F.Cu B.Cu) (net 1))
 (via (at 119.08 81.96) (size 0.5) (drill 0.3) (layers F.Cu B.Cu) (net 1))
 (via (at 119.08 81.39) (size 0.5) (drill 0.3) (layers F.Cu B.Cu) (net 1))
 (via (at 117.414999 81.335001) (size 0.5) (drill 0.3) (layers F.Cu B.Cu) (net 1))
 (via (at 118.13 81.67) (size 0.5) (drill 0.3) (layers F.Cu B.Cu) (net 1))
 (segment (start 116.96 69.73) (end 120.777 73.547) (width 0.5) (layer B.Cu) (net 1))
 (segment (start 120.777 79.023) (end 118.13 81.67) (width 0.5) (layer B.Cu) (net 1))
 (segment (start 120.777 73.547) (end 120.777 79.023) (width 0.5) (layer B.Cu) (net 1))
 (via (at 134.4422 75.3872) (size 0.8) (drill 0.4) (layers F.Cu B.Cu) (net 10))
 (via (at 133.378462 89.715862) (size 0.8) (drill 0.4) (layers F.Cu B.Cu) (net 10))
 (segment (start 134.4422 76.499798) (end 130.81 80.131998) (width 0.5) (layer B.Cu) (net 10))
 (segment (start 134.4422 75.3872) (end 134.4422 76.499798) (width 0.5) (layer B.Cu) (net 10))
 (segment (start 130.81 80.131998) (end 130.81 89.027) (width 0.5) (layer B.Cu) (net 10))
 (segment (start 131.498862 89.715862) (end 132.153138 89.715862) (width 0.5) (layer B.Cu) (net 10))
 (segment (start 130.81 89.027) (end 131.498862 89.715862) (width 0.5) (layer B.Cu) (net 10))
 (segment (start 132.153138 89.715862) (end 133.378462 89.715862) (width 0.5) (layer B.Cu) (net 10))
 (via (at 132.153138 89.715862) (size 0.8) (drill 0.4) (layers F.Cu B.Cu) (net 10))
 (segment (start 127.7874 77.0926) (end 126.72 78.16) (width 0.5) (layer F.Cu) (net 6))
 (segment (start 127.7874 75.3488) (end 127.7874 77.0926) (width 0.5) (layer F.Cu) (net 6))
 (via (at 124.73 77.53) (size 0.5) (drill 0.3) (layers F.Cu B.Cu) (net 5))
 (via (at 124.73 78.28) (size 0.5) (drill 0.3) (layers F.Cu B.Cu) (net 5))
 (via (at 124.73 78.95) (size 0.5) (drill 0.3) (layers F.Cu B.Cu) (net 5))
 (segment (start 125.5268 77.3532) (end 124.72 78.16) (width 0.5) (layer F.Cu) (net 5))
 (segment (start 125.5268 75.368) (end 125.5268 77.3532) (width 0.5) (layer F.Cu) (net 5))
 (segment (start 124.477599 74.318799) (end 125.5268 75.368) (width 0.5) (layer F.Cu) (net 5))
 (segment (start 120.961201 74.318799) (end 124.477599 74.318799) (width 0.5) (layer F.Cu) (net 5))
 (segment (start 120.07 75.21) (end 120.961201 74.318799) (width 0.5) (layer F.Cu) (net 5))
 (via (at 126.74972 64.046) (size 0.5) (drill 0.3) (layers F.Cu B.Cu) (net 12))
 (via (at 124.74972 65.046) (size 0.5) (drill 0.3) (layers F.Cu B.Cu) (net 12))
 (via (at 124.74972 63.046) (size 0.5) (drill 0.3) (layers F.Cu B.Cu) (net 12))
 (via (at 125.74972 63.046) (size 0.5) (drill 0.3) (layers F.Cu B.Cu) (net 12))
 (via (at 126.83 63.1) (size 0.5) (drill 0.3) (layers F.Cu B.Cu) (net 12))
 (via (at 124.74972 64.046) (size 0.5) (drill 0.3) (layers F.Cu B.Cu) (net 12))
 (via (at 125.7708 64.0092) (size 0.8) (drill 0.4) (layers F.Cu B.Cu) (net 12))
 (via (at 126.74972 65.046) (size 0.5) (drill 0.3) (layers F.Cu B.Cu) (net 12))
 (via (at 125.74972 65.046) (size 0.5) (drill 0.3) (layers F.Cu B.Cu) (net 12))
 (segment (start 122.35 56.38) (end 128.85 56.38) (width 0.5) (layer F.Cu) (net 12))
 (segment (start 127.040001 62.230001) (end 126.82 62.01) (width 0.5) (layer B.Cu) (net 12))
 (segment (start 130.091999 62.230001) (end 127.040001 62.230001) (width 0.5) (layer B.Cu) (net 12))
 (segment (start 131.632 60.69) (end 130.091999 62.230001) (width 0.5) (layer B.Cu) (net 12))
 (segment (start 126.82 58.41) (end 126.82 62.01) (width 0.5) (layer B.Cu) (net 12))
 (segment (start 128.85 56.38) (end 126.82 58.41) (width 0.5) (layer B.Cu) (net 12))
 (segment (start 119.32 61.911998) (end 121.922998 59.309) (width 0.5) (layer B.Cu) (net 12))
 (segment (start 119.32 64.04) (end 119.32 61.911998) (width 0.5) (layer B.Cu) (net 12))
 (segment (start 124.119 59.309) (end 126.82 62.01) (width 0.5) (layer B.Cu) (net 12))
 (segment (start 121.922998 59.309) (end 124.119 59.309) (width 0.5) (layer B.Cu) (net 12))
 (segment (start 125.7808 63.0492) (end 126.82 62.01) (width 0.5) (layer B.Cu) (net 12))
 (segment (start 125.7808 64.0842) (end 125.7808 63.0492) (width 0.5) (layer B.Cu) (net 12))
 (segment (start 128.98 64.17) (end 126.82 62.01) (width 0.5) (layer B.Cu) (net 12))
 (segment (start 130.98 64.17) (end 128.98 64.17) (width 0.5) (layer B.Cu) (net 12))
 (segment (start 133.135003 65.869999) (end 132.330001 65.869999) (width 0.5) (layer B.Cu) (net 13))
 (segment (start 134.099999 64.905003) (end 133.135003 65.869999) (width 0.5) (layer B.Cu) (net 13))
 (segment (start 134.099999 61.778001) (end 134.099999 64.905003) (width 0.5) (layer B.Cu) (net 13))
 (segment (start 132.330001 65.869999) (end 130.98 67.22) (width 0.5) (layer B.Cu) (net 13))
 (segment (start 135.188 60.69) (end 134.099999 61.778001) (width 0.5) (layer B.Cu) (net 13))
 (segment (start 130.048 76.832) (end 128.72 78.16) (width 0.5) (layer F.Cu) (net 7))
 (segment (start 130.048 75.3488) (end 130.048 76.832) (width 0.5) (layer F.Cu) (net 7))
 (segment (start 132.85 64.25) (end 132.85 64.25) (width 0.5) (layer F.Cu) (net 14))
 (segment (start 130.58501 66.64) (end 132.85 64.37501) (width 0.5) (layer F.Cu) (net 14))
 (via (at 132.85 64.37501) (size 0.8) (drill 0.4) (layers F.Cu B.Cu) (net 14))
 (segment (start 122.9 66.64) (end 130.58501 66.64) (width 0.5) (layer F.Cu) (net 14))
 (via (at 122.7836 78.2066) (size 0.5) (drill 0.3) (layers F.Cu B.Cu) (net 4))
 (segment (start 122.7836 68.2036) (end 122.7836 68.2036) (width 0.5) (layer B.Cu) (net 4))
 (segment (start 122.7836 78.2066) (end 122.7836 68.2036) (width 0.5) (layer B.Cu) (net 4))
 (segment (start 122.7836 68.2036) (end 121.22 66.64) (width 0.5) (layer B.Cu) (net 4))
 (via (at 122.7836 68.2036) (size 0.5) (drill 0.3) (layers F.Cu B.Cu) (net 4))
 (segment (start 123.0376 69.9499) (end 123.1575 69.83) (width 0.5) (layer F.Cu) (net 17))
 (segment (start 123.0376 73.0188) (end 123.0376 69.9499) (width 0.5) (layer F.Cu) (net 17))
 (segment (start 123.0376 75.8424) (end 120.72 78.16) (width 0.5) (layer F.Cu) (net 3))
 (segment (start 123.0376 75.4188) (end 123.0376 75.8424) (width 0.5) (layer F.Cu) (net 3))
 (segment (start 131.41 60.495) (end 131.45 60.535) (width 0.5) (layer F.Cu) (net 18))
 (segment (start 131.41 58.52) (end 131.41 60.495) (width 0.5) (layer F.Cu) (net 18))
 (via (at 121.33 64.13) (size 0.8) (drill 0.4) (layers F.Cu B.Cu) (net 16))
 (segment (start 122.35 63.09) (end 121.31 64.13) (width 0.5) (layer F.Cu) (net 16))
 (segment (start 122.35 60.88) (end 122.35 63.09) (width 0.5) (layer F.Cu) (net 16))
 (segment (start 122.35 60.88) (end 128.85 60.88) (width 0.5) (layer F.Cu) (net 16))
 (segment (start 128.85 58.68) (end 131.41 56.12) (width 0.5) (layer F.Cu) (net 16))
 (segment (start 128.85 60.88) (end 128.85 58.68) (width 0.5) (layer F.Cu) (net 16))
 (segment (start 131.41 56.12) (end 131.41 56.135) (width 0.5) (layer F.Cu) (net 16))
 (via (at 120.21 66.67) (size 0.8) (drill 0.4) (layers F.Cu B.Cu) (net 15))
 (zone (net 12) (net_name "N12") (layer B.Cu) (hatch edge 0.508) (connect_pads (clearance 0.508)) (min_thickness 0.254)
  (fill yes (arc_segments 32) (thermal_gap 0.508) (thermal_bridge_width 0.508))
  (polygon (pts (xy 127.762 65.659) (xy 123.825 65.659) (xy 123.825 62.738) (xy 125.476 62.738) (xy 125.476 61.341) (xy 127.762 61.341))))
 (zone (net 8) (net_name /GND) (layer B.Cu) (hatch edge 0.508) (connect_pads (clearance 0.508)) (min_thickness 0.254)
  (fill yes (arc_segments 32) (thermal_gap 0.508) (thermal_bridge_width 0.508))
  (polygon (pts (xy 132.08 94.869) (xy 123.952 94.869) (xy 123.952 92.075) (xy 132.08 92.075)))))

